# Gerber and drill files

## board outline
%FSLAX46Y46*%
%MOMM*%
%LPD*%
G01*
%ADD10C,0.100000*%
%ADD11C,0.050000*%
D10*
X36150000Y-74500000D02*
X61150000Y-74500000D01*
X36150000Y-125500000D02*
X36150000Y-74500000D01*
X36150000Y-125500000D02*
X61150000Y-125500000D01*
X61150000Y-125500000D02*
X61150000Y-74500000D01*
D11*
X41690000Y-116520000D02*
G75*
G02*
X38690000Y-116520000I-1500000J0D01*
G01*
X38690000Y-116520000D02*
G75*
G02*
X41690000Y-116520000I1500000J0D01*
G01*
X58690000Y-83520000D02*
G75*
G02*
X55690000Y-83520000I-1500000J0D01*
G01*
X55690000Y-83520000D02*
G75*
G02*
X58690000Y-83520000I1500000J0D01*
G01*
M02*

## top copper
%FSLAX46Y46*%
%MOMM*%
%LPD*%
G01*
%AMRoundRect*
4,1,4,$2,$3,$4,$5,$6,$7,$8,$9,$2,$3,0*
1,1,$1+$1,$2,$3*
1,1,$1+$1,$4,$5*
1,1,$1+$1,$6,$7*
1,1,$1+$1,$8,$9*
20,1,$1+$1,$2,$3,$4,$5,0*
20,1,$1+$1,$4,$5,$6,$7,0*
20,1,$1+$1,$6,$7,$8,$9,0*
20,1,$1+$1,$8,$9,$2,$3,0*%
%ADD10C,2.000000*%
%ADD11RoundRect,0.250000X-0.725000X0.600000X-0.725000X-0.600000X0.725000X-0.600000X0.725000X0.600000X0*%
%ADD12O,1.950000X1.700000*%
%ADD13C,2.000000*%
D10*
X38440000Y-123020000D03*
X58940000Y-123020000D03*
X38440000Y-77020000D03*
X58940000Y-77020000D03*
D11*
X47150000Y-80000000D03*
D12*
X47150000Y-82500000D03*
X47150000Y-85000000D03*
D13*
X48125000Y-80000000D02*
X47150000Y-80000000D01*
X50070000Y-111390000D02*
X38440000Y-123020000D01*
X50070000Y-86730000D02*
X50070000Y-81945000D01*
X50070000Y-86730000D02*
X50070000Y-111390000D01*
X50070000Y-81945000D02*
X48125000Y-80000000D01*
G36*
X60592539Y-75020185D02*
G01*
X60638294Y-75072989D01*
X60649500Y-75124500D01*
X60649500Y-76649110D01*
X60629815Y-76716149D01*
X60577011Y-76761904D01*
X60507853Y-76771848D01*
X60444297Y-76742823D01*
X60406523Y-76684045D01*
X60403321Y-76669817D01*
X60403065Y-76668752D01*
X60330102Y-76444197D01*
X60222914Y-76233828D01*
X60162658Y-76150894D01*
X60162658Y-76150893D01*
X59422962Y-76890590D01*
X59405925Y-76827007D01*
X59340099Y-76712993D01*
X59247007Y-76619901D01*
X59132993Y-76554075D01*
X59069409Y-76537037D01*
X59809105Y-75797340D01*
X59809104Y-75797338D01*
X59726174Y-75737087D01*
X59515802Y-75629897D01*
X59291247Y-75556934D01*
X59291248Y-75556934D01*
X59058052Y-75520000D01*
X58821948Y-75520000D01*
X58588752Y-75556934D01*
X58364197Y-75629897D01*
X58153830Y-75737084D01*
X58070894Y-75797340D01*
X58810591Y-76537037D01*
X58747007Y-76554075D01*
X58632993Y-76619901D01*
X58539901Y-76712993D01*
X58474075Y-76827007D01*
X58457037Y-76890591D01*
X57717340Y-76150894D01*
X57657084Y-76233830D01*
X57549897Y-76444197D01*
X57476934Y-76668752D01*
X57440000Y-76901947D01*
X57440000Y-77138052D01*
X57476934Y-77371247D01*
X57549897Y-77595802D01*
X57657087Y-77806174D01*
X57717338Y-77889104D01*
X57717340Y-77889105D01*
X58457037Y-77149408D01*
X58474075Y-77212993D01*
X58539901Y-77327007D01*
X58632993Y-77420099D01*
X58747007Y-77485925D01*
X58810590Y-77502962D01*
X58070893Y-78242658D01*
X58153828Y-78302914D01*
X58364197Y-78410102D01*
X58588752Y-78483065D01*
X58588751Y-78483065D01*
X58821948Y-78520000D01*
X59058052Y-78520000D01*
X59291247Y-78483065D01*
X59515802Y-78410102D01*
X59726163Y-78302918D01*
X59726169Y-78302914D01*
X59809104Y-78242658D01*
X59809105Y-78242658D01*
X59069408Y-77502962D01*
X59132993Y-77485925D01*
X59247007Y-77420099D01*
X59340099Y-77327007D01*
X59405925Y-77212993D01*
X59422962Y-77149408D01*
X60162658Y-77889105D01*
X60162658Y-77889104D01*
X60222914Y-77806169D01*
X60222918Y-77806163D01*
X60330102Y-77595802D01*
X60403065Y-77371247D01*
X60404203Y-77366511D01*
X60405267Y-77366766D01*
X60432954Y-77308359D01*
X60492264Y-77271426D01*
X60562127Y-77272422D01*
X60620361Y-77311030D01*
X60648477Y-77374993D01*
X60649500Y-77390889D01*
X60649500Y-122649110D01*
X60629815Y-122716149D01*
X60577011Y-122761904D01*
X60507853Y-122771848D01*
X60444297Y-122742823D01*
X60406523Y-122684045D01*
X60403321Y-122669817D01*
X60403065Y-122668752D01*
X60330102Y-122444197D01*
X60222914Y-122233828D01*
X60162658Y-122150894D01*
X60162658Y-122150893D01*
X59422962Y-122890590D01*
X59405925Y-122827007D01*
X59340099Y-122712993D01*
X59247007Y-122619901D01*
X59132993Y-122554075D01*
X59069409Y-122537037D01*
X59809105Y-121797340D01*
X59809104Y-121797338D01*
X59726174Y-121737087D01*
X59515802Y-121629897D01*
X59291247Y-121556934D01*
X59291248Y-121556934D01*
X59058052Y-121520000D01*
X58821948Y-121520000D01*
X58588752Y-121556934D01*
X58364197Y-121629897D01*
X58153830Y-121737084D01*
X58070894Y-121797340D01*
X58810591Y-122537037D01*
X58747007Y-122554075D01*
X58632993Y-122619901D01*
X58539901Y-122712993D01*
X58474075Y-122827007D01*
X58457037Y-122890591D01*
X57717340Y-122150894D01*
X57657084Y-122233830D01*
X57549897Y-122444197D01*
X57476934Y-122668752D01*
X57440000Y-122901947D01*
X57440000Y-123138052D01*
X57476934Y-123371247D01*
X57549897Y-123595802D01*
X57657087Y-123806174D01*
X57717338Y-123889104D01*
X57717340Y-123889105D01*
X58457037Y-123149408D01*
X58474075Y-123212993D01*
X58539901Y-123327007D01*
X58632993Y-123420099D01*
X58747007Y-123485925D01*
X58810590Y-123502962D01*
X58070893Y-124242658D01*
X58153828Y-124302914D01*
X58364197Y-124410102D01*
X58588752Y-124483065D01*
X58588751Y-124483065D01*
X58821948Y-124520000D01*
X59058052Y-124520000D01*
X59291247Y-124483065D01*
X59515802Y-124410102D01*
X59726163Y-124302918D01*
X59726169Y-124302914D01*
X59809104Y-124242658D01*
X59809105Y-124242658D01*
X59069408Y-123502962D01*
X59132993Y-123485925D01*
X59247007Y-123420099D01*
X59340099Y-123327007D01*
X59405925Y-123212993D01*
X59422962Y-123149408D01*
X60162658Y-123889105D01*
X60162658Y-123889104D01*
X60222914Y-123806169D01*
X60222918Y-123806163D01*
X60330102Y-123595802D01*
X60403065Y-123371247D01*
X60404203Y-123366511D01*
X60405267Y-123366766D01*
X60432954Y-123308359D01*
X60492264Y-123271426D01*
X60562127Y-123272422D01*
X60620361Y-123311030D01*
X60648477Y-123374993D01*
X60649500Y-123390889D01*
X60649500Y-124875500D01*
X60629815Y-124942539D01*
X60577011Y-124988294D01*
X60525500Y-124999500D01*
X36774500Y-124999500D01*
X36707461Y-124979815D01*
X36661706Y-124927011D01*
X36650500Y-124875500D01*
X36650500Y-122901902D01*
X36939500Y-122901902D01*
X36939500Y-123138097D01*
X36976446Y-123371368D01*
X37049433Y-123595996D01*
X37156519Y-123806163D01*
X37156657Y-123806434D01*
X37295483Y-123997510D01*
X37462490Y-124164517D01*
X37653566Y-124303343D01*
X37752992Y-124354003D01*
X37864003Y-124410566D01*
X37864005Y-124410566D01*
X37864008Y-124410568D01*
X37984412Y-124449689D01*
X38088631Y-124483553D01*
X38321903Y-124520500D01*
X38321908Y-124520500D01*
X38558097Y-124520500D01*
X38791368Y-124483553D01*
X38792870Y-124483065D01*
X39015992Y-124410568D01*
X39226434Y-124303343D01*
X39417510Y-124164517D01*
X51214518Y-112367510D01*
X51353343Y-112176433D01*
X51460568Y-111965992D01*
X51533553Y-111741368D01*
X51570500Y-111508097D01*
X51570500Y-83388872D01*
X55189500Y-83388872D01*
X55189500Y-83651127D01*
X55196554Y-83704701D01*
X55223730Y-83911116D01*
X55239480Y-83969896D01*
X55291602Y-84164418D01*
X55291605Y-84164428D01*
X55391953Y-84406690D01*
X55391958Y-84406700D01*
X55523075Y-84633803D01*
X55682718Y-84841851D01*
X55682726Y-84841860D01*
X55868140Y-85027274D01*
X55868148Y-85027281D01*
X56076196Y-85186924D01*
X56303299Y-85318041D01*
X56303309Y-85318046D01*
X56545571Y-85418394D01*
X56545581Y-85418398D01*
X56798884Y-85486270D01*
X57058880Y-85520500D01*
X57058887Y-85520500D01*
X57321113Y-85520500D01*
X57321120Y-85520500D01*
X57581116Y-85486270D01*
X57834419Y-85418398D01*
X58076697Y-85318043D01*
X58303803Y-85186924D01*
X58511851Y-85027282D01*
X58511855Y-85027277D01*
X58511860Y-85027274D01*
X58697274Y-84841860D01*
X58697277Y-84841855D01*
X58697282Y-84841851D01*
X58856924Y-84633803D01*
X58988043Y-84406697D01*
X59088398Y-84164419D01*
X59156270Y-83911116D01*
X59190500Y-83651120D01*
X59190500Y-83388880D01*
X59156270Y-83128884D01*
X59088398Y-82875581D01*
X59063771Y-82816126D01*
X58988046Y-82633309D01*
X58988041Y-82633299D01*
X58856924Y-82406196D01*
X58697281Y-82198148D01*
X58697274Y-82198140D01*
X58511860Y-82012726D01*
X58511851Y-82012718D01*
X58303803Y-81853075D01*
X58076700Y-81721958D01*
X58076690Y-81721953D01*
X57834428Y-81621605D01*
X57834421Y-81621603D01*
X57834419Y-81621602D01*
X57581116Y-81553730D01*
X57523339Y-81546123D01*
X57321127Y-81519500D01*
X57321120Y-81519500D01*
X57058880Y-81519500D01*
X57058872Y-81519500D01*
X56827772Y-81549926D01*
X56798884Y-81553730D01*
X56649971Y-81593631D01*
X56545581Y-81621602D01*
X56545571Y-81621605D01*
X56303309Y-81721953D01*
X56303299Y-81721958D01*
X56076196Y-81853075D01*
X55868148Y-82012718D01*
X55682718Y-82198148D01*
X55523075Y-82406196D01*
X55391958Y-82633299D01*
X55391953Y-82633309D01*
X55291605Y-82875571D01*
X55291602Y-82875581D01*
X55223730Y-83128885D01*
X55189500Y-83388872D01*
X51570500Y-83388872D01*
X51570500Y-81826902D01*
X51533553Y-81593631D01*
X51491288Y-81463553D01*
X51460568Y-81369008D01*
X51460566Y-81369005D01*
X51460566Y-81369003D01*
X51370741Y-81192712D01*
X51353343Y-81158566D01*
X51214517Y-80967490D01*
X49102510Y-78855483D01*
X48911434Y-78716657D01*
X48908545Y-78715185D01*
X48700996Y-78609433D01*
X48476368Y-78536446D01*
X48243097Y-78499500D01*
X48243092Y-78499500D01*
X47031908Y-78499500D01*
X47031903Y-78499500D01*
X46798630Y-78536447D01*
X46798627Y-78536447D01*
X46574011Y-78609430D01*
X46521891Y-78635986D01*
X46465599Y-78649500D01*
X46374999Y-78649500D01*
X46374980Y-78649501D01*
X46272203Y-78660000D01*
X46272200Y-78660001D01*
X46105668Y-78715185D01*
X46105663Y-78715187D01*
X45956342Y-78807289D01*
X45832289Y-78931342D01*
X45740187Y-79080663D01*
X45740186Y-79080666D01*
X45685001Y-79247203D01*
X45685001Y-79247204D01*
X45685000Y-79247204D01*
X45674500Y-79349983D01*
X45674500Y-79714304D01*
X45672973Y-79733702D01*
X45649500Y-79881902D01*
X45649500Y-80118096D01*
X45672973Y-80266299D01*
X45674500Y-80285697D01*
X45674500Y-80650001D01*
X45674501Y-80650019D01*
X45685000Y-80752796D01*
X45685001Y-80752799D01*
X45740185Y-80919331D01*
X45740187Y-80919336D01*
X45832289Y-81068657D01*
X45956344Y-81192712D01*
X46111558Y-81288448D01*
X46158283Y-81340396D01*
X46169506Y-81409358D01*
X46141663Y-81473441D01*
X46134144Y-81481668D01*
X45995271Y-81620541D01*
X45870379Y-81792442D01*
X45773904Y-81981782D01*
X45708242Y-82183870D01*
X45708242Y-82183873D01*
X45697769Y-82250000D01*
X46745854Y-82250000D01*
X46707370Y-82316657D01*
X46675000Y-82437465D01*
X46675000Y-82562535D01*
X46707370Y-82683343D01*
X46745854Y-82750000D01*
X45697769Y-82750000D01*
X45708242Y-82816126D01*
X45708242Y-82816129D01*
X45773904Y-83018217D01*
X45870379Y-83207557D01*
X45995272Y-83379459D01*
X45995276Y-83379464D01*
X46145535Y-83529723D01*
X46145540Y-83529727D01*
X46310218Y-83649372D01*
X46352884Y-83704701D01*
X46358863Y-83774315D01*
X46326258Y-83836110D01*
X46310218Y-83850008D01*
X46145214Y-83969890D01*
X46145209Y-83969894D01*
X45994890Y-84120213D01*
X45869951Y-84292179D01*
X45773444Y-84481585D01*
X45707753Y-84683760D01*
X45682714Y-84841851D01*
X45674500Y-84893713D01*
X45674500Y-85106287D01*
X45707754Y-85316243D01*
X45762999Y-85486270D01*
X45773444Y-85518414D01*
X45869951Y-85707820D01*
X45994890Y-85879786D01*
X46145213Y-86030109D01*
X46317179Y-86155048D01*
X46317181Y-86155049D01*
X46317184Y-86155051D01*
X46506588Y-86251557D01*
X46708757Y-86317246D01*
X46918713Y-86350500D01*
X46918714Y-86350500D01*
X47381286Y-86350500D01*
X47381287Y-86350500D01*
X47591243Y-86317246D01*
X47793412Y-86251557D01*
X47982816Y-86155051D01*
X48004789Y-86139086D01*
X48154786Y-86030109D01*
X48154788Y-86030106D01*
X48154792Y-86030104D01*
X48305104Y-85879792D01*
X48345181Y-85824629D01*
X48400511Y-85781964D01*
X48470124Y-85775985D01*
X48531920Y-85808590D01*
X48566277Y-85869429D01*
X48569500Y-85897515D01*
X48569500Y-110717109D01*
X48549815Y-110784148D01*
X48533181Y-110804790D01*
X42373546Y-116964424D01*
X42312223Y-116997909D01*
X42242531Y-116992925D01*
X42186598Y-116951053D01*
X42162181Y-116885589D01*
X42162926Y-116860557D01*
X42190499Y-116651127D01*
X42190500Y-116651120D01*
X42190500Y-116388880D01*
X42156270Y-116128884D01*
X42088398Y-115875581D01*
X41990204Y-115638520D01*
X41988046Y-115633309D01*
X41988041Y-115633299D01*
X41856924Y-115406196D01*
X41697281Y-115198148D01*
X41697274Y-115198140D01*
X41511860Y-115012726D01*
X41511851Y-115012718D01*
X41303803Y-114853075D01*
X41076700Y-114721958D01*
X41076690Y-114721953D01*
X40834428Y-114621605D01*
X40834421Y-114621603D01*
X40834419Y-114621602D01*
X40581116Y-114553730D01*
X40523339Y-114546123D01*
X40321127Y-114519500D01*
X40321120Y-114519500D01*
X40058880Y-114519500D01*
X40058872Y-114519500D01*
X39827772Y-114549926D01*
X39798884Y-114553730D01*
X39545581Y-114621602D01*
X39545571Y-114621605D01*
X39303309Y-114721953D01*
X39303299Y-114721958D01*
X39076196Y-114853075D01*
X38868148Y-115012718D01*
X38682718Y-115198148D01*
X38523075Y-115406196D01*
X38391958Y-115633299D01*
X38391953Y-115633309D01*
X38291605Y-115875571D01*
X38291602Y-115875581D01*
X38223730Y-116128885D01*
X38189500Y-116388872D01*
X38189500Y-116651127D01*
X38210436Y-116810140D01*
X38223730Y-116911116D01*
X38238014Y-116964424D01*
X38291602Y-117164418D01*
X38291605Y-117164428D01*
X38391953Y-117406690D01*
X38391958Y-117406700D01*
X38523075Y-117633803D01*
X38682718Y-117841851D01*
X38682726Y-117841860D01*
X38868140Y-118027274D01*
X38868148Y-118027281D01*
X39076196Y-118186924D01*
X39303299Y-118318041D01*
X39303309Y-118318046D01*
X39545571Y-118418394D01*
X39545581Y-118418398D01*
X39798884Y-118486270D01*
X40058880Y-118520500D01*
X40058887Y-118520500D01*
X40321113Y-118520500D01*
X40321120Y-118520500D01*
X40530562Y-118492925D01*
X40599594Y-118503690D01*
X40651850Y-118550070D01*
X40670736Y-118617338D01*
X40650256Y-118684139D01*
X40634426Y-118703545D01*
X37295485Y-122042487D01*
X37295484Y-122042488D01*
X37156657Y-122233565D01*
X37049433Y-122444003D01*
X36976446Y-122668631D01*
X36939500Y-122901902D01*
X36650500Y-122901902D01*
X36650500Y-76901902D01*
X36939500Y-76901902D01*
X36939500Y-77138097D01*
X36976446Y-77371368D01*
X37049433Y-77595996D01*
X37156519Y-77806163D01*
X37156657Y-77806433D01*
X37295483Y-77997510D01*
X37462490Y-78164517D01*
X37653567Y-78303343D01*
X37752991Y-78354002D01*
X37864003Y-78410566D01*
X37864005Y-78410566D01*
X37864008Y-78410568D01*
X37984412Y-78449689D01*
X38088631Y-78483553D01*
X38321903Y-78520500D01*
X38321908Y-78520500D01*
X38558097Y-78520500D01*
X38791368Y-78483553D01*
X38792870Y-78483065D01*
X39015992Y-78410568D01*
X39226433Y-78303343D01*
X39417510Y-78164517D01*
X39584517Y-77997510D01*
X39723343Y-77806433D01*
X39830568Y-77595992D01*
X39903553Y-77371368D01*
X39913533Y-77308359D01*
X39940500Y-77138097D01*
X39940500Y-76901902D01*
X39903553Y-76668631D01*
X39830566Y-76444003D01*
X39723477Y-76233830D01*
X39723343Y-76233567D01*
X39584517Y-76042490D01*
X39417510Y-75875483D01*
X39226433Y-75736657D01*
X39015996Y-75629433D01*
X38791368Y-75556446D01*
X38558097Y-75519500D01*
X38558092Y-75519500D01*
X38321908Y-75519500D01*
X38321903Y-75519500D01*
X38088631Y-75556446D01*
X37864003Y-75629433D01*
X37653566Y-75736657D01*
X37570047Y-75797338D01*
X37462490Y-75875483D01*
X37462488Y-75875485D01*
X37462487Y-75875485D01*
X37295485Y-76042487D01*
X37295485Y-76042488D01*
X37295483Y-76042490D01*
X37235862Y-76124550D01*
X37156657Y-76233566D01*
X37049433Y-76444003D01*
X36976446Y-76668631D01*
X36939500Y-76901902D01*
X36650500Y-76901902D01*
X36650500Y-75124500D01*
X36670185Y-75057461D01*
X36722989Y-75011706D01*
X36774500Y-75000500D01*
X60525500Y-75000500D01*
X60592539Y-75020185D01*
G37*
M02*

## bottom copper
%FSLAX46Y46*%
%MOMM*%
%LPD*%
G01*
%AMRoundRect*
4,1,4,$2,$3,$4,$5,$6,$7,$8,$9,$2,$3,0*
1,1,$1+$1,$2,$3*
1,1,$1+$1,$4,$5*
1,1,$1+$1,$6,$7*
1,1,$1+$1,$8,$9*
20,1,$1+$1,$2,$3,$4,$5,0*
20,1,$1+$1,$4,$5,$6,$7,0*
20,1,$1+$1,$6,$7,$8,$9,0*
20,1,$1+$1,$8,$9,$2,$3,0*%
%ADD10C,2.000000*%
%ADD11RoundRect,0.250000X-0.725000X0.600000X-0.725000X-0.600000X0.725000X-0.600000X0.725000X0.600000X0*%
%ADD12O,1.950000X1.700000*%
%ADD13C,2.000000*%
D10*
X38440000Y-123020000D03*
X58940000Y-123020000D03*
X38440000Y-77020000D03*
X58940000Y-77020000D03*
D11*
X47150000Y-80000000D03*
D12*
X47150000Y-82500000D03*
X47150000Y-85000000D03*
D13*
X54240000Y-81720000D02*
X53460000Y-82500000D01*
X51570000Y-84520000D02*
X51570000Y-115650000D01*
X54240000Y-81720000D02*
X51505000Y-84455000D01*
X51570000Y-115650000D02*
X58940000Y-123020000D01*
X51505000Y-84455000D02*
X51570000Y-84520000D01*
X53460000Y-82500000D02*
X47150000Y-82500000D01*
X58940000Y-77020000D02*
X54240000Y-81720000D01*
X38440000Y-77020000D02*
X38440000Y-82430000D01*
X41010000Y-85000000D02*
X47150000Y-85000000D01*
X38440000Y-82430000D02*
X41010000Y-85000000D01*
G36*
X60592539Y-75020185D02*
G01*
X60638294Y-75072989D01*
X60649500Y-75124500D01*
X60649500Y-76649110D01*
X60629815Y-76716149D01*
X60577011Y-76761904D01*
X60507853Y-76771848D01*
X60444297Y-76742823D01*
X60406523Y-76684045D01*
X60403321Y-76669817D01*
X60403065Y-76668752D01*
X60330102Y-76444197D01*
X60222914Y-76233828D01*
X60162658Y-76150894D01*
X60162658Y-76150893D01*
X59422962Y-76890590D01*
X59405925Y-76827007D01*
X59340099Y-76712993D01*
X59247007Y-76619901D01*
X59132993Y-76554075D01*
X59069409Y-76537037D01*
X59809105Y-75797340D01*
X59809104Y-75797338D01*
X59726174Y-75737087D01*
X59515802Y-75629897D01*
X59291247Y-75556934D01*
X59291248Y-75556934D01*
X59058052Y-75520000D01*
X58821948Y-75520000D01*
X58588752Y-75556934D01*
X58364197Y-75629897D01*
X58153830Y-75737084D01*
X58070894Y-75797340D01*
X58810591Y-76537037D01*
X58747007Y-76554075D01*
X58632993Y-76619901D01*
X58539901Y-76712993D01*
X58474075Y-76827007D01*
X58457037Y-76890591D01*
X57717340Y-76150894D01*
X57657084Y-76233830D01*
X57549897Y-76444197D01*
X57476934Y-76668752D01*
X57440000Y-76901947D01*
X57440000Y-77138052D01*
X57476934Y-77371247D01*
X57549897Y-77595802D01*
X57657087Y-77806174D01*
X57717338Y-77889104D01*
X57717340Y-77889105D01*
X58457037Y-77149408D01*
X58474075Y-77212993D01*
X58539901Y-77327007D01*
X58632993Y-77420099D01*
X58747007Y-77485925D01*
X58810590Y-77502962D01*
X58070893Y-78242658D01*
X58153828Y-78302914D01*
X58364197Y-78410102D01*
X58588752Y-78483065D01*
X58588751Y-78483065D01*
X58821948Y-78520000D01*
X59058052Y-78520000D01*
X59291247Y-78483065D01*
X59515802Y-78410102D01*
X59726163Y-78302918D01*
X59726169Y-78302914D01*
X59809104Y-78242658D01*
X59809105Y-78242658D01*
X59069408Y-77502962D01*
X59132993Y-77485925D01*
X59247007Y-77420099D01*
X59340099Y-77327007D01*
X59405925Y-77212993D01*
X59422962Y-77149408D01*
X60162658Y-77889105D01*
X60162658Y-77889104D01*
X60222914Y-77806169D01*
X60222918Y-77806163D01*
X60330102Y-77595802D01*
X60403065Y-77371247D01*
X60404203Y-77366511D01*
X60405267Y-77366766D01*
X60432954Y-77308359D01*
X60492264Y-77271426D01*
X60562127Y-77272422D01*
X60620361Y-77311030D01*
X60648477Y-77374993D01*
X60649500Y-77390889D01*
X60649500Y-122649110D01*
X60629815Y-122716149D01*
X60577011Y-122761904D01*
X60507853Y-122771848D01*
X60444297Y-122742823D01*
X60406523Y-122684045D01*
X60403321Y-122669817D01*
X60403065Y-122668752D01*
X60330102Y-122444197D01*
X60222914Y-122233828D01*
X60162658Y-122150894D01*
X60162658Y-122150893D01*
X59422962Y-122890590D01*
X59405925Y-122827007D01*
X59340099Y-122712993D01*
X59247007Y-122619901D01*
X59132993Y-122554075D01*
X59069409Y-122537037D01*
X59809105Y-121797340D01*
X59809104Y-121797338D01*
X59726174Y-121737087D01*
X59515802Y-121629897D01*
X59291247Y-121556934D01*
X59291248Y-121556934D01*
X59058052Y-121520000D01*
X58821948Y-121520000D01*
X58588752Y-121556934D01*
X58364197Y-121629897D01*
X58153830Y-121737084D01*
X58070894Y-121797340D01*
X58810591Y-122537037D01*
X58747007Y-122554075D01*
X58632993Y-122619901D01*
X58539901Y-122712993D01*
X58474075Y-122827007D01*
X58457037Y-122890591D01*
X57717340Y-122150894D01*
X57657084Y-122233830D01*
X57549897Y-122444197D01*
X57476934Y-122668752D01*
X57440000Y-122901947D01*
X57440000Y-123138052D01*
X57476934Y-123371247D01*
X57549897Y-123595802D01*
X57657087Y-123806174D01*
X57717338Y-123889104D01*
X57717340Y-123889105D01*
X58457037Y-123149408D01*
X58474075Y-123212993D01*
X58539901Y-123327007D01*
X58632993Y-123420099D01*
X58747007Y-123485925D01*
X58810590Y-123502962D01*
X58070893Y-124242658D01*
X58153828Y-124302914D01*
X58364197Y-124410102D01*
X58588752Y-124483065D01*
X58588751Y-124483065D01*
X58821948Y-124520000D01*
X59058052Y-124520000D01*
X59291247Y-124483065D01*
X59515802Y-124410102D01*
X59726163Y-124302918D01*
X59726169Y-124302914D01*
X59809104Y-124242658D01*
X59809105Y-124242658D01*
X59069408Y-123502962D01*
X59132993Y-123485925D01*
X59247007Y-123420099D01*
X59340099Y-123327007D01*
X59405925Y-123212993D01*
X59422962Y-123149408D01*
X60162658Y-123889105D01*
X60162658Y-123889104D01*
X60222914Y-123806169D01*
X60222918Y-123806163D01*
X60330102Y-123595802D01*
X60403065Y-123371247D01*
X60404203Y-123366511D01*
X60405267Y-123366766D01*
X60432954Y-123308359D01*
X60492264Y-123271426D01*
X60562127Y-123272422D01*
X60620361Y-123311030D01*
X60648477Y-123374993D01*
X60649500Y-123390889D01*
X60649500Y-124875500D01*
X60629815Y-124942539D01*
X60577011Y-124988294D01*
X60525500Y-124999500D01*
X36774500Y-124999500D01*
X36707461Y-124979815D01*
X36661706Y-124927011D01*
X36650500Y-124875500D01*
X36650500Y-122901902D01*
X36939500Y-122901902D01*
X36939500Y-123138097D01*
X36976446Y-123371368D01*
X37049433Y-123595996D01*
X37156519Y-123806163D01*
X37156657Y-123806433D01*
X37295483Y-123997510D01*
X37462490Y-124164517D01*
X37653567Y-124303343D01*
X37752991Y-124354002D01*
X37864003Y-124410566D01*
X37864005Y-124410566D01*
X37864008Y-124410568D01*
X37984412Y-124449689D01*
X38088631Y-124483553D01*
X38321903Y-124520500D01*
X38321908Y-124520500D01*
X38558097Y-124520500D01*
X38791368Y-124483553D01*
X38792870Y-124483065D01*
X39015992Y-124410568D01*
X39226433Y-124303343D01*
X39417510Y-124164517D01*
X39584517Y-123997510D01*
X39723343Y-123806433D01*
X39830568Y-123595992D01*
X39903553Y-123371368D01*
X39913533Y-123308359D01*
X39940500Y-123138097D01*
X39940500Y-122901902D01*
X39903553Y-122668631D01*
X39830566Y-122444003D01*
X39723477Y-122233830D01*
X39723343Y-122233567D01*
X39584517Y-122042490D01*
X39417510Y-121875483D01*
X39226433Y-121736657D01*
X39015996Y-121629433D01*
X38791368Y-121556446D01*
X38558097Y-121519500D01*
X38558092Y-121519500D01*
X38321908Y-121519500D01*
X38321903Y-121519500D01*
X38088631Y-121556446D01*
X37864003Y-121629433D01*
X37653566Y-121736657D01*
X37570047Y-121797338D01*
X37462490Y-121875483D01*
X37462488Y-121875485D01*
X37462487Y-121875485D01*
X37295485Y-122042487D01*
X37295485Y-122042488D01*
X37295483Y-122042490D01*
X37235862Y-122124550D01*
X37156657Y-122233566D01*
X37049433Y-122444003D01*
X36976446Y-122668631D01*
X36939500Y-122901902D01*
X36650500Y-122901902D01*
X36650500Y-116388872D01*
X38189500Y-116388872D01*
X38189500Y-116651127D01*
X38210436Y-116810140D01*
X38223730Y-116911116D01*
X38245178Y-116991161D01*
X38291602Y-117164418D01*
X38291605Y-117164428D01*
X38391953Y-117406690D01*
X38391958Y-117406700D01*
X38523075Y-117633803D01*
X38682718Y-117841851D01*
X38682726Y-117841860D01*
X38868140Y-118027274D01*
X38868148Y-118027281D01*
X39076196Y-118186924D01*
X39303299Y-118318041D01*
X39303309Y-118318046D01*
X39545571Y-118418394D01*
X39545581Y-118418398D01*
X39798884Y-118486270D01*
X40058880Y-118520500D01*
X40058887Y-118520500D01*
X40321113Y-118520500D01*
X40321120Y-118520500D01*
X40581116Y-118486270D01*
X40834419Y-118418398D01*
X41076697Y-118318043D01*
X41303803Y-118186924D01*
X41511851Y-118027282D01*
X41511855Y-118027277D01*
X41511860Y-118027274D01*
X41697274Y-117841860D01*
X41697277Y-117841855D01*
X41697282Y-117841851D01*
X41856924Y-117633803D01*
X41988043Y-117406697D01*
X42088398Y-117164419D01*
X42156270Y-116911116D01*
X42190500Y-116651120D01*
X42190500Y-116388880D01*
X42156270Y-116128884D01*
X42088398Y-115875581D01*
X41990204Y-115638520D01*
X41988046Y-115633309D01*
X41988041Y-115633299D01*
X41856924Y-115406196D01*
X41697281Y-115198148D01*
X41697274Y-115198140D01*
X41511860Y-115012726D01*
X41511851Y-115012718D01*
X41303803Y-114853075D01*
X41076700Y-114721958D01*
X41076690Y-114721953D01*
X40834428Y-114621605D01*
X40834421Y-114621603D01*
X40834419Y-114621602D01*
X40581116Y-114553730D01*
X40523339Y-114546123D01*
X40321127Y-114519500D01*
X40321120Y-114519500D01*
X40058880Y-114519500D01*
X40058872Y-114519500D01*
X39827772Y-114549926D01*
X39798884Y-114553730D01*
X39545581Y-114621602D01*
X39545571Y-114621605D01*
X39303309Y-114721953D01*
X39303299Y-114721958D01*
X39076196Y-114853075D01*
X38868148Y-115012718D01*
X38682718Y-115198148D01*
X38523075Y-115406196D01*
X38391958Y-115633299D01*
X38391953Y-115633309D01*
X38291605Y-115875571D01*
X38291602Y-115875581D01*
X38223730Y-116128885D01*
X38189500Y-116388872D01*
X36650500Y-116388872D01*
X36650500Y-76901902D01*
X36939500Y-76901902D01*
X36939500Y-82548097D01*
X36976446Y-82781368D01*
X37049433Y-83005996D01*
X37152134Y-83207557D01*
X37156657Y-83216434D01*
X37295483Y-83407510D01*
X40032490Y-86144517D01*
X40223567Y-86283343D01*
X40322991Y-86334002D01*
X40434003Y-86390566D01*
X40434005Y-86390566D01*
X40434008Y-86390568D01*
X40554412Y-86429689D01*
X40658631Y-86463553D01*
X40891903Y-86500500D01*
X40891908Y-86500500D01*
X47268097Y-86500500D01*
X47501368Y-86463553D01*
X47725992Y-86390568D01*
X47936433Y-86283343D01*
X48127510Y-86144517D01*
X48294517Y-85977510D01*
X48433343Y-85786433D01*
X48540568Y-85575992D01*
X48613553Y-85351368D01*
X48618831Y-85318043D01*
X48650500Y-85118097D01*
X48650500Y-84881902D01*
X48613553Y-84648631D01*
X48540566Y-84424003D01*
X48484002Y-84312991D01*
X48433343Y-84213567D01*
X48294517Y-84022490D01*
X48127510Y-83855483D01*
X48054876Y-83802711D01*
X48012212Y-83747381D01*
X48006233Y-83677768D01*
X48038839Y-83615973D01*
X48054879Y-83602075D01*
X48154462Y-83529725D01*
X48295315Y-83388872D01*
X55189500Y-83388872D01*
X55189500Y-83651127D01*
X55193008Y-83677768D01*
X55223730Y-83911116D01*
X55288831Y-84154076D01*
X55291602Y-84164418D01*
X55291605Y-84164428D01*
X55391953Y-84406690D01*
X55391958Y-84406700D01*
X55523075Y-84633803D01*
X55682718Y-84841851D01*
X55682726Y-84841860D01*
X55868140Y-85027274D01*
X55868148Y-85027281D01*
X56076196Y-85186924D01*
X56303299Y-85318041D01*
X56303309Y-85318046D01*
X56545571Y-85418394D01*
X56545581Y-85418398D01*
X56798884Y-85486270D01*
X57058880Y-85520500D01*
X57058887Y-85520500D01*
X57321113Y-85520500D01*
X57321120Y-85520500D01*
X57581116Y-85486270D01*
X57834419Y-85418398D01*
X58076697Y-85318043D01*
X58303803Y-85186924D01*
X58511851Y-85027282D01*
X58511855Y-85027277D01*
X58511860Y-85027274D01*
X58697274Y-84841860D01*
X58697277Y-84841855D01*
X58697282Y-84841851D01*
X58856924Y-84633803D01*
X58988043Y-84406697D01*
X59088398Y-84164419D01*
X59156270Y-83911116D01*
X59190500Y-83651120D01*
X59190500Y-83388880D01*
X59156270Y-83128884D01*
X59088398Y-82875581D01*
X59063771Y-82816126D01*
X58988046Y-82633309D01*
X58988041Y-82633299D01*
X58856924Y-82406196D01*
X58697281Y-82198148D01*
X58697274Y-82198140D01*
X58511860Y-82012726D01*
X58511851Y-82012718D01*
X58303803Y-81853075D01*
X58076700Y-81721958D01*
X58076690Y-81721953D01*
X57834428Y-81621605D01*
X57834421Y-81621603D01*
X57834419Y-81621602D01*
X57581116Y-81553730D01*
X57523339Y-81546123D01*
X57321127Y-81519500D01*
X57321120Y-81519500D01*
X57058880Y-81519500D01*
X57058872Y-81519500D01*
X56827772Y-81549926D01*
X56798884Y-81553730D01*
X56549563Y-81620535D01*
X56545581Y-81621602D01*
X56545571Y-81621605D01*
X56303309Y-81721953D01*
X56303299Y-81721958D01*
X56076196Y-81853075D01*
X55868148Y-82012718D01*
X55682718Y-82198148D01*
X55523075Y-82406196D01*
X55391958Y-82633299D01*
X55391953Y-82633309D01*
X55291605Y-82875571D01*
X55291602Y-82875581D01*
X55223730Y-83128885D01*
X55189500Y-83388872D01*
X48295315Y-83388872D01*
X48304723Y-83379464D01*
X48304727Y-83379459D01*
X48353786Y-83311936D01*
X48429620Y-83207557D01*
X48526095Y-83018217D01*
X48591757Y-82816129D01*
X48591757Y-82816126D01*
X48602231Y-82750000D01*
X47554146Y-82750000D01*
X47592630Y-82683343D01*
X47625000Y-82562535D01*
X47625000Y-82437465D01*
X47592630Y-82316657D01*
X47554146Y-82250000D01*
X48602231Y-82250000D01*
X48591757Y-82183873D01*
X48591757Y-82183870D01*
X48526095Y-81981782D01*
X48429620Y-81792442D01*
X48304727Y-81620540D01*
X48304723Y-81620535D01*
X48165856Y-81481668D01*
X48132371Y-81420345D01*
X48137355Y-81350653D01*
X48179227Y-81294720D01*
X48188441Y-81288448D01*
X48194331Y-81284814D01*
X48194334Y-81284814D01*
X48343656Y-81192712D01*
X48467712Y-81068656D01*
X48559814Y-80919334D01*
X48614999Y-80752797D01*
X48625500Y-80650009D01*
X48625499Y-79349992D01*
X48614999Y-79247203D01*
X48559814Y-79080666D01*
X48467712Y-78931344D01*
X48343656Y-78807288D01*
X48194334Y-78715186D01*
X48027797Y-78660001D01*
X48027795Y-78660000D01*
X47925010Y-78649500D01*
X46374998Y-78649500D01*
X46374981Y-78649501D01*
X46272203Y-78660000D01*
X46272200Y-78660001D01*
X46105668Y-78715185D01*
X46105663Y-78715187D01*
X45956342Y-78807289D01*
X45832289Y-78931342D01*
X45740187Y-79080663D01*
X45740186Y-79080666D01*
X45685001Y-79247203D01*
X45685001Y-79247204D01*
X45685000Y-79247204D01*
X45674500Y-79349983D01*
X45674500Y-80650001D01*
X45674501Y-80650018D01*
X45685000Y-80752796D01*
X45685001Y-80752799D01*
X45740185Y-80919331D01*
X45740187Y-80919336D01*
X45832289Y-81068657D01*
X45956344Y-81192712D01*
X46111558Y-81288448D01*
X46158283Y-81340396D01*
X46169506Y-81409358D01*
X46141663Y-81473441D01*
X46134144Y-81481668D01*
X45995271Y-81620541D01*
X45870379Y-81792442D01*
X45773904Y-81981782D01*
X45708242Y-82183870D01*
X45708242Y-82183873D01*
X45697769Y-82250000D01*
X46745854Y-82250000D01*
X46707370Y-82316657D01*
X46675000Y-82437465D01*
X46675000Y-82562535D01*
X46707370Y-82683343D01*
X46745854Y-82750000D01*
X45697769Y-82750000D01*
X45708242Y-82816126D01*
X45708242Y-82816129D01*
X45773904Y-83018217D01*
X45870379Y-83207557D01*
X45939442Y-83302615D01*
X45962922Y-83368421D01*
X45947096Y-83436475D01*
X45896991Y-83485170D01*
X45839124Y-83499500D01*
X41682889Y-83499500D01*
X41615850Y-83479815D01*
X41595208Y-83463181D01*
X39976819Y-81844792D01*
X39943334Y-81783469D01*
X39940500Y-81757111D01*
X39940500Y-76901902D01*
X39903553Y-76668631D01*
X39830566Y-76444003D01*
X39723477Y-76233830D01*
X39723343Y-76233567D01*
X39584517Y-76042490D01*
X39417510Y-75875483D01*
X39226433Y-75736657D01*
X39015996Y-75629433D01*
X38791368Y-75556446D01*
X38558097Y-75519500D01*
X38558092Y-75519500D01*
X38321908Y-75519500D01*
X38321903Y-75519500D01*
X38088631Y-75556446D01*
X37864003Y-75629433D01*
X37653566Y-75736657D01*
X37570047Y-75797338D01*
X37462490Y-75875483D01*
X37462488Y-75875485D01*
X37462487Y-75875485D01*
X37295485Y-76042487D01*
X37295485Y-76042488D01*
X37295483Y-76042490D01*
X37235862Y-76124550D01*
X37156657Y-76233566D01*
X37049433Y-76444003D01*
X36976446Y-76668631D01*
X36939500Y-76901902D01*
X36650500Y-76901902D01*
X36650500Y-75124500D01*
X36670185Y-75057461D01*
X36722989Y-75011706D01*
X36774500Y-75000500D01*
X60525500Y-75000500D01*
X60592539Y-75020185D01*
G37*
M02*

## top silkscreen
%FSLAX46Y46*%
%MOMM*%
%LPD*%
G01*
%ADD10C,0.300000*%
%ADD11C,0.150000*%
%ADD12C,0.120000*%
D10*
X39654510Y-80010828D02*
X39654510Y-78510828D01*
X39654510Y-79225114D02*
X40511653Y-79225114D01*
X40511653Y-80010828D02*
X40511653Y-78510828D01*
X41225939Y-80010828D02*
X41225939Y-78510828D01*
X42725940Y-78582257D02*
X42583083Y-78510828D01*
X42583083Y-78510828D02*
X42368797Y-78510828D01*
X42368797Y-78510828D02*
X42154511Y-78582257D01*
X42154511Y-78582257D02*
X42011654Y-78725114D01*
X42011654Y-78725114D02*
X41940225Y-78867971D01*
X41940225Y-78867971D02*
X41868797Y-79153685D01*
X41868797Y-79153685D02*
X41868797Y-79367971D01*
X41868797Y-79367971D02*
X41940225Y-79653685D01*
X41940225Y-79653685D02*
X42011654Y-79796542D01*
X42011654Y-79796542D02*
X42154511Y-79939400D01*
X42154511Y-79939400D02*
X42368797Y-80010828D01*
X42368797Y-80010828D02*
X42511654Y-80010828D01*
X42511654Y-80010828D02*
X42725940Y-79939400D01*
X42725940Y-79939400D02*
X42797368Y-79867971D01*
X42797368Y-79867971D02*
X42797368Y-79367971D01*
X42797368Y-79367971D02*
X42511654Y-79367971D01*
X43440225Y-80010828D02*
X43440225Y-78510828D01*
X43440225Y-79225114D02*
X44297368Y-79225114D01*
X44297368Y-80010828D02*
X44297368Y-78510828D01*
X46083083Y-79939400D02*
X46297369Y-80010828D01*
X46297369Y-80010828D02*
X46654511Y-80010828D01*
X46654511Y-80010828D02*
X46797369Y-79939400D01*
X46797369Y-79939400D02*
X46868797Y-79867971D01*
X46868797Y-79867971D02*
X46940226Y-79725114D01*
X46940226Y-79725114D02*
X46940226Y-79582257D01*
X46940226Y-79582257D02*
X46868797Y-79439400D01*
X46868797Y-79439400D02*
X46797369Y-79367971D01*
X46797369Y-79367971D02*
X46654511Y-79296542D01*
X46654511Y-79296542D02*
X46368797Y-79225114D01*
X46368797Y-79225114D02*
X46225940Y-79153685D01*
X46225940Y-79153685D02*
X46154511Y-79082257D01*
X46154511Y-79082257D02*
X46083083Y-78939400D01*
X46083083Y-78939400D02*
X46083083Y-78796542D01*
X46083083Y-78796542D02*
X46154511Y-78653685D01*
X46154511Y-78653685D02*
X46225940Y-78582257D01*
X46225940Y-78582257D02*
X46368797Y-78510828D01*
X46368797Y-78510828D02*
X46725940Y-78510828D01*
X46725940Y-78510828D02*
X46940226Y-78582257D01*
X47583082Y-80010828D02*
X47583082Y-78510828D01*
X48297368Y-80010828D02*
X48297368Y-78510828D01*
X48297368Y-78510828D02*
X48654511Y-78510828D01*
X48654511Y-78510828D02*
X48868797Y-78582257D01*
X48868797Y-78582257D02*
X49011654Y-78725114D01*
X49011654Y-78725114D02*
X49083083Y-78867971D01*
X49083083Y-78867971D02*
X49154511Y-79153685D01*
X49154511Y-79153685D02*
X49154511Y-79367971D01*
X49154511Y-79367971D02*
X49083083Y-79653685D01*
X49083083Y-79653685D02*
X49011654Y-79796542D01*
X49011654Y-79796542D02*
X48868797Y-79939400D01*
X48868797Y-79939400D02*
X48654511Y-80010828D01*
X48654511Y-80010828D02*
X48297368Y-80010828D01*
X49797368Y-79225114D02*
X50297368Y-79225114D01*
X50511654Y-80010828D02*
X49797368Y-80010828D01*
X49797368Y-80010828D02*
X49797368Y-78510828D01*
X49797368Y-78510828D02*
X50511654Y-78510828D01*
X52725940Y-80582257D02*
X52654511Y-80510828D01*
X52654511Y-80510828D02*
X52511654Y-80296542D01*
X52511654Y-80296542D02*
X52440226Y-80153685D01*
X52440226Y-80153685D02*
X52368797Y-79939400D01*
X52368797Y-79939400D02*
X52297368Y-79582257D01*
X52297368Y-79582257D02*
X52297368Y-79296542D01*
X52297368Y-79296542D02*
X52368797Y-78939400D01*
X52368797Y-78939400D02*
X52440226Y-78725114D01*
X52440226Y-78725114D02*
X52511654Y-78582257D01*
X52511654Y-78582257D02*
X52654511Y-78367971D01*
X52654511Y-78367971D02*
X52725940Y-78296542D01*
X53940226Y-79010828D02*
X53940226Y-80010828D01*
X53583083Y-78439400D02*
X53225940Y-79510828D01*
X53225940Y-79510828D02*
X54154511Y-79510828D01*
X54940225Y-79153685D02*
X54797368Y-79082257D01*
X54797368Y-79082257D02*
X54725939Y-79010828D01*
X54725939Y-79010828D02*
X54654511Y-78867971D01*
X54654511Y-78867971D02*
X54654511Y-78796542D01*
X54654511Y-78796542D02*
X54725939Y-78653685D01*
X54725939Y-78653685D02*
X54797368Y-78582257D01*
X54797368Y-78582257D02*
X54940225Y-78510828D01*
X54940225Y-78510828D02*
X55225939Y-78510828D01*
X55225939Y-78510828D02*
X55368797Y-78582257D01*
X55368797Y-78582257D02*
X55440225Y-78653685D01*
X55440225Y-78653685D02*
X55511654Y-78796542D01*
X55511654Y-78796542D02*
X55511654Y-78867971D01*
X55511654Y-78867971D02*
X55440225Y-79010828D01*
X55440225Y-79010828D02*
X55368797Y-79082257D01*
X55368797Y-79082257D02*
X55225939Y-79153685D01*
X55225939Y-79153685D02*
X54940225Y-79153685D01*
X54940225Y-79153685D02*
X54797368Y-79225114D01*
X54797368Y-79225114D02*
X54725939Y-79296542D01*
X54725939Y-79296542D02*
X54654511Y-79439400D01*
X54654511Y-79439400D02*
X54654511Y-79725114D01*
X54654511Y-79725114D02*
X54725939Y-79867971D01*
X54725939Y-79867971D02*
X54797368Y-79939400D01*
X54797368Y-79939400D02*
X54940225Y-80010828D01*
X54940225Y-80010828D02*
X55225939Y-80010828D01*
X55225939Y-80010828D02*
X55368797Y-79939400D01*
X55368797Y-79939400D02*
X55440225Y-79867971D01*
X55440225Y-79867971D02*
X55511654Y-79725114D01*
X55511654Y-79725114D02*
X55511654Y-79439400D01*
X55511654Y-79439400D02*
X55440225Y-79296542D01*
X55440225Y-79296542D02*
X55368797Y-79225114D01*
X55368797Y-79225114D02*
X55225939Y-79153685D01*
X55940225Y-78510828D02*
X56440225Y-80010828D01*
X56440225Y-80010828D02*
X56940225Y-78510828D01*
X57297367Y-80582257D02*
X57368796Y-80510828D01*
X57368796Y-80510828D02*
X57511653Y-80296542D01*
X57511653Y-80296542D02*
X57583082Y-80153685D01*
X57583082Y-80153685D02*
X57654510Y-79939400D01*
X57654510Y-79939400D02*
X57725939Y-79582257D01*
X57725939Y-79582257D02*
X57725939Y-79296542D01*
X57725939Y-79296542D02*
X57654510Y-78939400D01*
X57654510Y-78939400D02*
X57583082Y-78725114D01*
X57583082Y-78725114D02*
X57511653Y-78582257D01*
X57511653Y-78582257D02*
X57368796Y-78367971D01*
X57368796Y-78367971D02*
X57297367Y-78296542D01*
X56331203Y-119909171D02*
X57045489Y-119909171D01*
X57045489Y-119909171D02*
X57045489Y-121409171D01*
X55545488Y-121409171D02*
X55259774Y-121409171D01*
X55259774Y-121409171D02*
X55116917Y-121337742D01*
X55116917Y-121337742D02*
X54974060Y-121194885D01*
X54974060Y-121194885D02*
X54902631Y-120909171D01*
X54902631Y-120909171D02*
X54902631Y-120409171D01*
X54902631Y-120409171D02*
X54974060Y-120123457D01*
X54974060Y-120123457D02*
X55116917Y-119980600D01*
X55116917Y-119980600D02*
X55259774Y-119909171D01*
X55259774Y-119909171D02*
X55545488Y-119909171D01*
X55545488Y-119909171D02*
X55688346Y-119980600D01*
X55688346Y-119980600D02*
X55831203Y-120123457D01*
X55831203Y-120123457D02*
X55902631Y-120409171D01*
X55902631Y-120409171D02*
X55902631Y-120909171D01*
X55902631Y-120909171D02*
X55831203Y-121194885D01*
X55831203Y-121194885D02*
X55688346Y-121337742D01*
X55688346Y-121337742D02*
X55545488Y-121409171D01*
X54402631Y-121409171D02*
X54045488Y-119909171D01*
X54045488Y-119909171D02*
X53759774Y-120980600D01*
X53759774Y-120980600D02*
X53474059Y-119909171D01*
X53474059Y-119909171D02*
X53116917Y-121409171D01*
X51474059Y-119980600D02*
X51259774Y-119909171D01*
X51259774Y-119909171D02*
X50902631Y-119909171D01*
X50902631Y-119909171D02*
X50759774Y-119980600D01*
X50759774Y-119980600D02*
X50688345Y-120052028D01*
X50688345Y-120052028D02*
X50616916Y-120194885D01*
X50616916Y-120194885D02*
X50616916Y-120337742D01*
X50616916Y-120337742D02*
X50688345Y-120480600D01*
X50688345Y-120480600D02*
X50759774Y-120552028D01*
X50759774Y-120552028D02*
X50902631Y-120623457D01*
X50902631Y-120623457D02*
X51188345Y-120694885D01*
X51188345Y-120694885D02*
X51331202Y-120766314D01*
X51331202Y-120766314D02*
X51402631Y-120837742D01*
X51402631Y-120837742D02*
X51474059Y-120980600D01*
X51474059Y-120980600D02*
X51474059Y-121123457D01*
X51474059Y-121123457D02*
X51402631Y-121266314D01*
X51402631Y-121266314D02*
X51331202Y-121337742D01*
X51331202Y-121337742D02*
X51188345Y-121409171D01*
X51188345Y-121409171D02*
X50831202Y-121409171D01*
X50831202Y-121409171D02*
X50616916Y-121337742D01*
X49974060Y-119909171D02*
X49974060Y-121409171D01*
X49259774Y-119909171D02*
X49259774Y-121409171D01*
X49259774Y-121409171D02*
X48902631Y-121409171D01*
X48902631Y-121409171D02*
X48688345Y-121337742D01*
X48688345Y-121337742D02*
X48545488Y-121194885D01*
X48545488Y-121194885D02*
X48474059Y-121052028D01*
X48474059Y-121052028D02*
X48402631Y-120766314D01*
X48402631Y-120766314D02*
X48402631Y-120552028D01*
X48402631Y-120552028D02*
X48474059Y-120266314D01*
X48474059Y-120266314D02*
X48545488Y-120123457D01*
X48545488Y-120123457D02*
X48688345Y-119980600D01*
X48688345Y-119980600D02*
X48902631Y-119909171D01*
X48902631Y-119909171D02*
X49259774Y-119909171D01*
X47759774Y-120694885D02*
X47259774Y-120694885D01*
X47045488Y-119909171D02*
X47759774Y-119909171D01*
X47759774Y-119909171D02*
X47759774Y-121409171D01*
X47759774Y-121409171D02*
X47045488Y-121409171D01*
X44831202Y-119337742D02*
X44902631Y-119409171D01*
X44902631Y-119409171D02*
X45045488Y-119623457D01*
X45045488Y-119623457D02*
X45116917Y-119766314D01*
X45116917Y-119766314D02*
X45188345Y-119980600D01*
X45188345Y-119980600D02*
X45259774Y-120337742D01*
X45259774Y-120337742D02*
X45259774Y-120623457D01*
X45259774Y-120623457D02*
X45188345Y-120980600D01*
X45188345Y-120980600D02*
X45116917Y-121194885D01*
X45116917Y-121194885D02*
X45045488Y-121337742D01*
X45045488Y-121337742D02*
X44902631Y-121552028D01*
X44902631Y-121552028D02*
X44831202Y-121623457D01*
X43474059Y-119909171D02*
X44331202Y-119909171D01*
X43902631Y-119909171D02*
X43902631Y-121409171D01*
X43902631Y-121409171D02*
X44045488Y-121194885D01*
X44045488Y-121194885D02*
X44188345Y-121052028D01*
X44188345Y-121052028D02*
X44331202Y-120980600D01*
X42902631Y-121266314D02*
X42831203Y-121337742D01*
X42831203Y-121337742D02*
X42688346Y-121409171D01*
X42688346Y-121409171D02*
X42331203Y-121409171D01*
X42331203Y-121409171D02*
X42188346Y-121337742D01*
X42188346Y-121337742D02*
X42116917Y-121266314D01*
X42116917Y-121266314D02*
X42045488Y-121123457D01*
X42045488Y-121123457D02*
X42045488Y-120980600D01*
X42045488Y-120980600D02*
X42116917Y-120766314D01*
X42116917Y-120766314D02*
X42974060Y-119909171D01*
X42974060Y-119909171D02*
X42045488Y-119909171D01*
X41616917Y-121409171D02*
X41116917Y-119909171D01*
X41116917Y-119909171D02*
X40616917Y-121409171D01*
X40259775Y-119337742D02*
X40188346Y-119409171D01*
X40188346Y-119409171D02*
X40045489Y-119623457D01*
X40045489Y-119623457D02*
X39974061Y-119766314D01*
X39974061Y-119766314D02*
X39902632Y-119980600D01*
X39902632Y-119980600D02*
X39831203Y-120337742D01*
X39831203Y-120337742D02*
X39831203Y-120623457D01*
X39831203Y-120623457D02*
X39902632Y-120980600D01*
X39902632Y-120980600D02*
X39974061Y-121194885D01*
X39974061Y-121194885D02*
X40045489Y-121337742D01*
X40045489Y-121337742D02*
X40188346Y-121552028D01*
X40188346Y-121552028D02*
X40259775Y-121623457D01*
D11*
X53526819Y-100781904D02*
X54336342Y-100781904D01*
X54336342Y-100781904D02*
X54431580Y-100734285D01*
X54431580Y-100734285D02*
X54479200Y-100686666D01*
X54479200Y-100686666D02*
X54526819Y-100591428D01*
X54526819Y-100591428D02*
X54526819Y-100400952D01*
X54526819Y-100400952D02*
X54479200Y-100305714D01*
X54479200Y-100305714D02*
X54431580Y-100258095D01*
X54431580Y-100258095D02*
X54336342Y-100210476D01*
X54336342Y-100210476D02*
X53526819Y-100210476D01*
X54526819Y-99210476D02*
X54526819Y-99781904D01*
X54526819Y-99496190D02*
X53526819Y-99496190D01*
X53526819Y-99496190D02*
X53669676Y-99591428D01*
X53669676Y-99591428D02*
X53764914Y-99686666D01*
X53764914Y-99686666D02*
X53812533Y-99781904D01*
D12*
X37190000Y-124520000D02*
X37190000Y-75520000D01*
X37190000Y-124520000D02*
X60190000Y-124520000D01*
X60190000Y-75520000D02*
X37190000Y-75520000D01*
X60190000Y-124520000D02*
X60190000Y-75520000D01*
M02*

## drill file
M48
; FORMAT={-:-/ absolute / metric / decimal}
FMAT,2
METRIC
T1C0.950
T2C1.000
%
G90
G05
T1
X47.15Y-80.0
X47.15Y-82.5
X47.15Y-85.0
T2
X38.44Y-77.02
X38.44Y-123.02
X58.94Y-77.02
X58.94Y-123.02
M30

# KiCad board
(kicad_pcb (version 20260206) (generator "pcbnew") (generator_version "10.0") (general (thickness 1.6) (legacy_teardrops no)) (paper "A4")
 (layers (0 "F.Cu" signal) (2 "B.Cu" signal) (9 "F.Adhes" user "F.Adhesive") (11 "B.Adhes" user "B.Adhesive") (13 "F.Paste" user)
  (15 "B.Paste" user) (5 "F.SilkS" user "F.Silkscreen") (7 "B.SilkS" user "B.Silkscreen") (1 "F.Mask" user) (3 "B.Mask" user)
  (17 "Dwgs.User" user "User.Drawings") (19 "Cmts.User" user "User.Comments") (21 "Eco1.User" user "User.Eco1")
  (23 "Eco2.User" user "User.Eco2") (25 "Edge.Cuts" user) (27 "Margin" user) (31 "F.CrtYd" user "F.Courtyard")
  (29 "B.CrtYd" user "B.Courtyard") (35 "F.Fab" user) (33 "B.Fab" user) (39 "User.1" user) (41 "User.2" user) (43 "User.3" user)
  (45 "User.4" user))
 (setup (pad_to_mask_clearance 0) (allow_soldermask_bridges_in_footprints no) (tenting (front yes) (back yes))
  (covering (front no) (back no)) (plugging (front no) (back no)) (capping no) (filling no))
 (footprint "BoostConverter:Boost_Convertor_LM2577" (layer "F.Cu") (at 48.69 100.02 90)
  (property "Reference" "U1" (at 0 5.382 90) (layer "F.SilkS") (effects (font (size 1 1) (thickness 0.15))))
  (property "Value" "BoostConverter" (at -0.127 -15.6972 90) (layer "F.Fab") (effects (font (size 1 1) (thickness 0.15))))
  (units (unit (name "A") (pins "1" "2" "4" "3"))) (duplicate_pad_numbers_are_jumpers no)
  (fp_line (start -24.5 -11.5) (end 24.5 -11.5) (stroke (width 0.12) (type solid)) (layer "F.SilkS"))
  (fp_line (start -24.5 -11.5) (end -24.5 11.5) (stroke (width 0.12) (type solid)) (layer "F.SilkS"))
  (fp_line (start 24.5 11.5) (end 24.5 -11.5) (stroke (width 0.12) (type solid)) (layer "F.SilkS"))
  (fp_line (start -24.5 11.5) (end 24.5 11.5) (stroke (width 0.12) (type solid)) (layer "F.SilkS"))
  (fp_circle (center -16.5 -8.5) (end -15 -8.5) (stroke (width 0.05) (type default)) (fill no) (layer "Edge.Cuts"))
  (fp_circle (center 16.5 8.5) (end 18 8.5) (stroke (width 0.05) (type default)) (fill no) (layer "Edge.Cuts"))
  (pad "1" thru_hole circle (at -23 -10.25 90) (size 2 2) (drill 1) (layers "*.Cu" "*.Mask") (remove_unused_layers no) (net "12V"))
  (pad "2" thru_hole circle (at -23 10.25 90) (size 2 2) (drill 1) (layers "*.Cu" "*.Mask") (remove_unused_layers no) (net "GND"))
  (pad "3" thru_hole circle (at 23 -10.25 90) (size 2 2) (drill 1) (layers "*.Cu" "*.Mask") (remove_unused_layers no) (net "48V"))
  (pad "4" thru_hole circle (at 23 10.25 90) (size 2 2) (drill 1) (layers "*.Cu" "*.Mask") (remove_unused_layers no) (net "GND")))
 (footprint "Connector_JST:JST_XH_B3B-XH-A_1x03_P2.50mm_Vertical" (layer "B.Cu") (at 47.15 80 -90)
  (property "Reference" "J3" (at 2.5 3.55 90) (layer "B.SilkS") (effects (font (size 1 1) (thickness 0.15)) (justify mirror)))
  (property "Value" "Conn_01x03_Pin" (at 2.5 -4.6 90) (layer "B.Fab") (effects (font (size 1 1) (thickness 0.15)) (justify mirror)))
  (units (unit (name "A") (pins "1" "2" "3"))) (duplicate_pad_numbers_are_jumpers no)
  (pad "1" thru_hole roundrect (at 0 0 270) (size 1.7 1.95) (drill 0.95) (layers "*.Cu" "*.Mask") (remove_unused_layers no)
   (roundrect_rratio 0.147059) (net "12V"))
  (pad "2" thru_hole oval (at 2.5 0 270) (size 1.7 1.95) (drill 0.95) (layers "*.Cu" "*.Mask") (remove_unused_layers no) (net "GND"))
  (pad "3" thru_hole oval (at 5 0 270) (size 1.7 1.95) (drill 0.95) (layers "*.Cu" "*.Mask") (remove_unused_layers no) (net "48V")))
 (gr_line (start 36.15 74.5) (end 61.15 74.5) (stroke (width 0.1) (type default)) (layer "Edge.Cuts"))
 (gr_line (start 36.15 125.5) (end 36.15 74.5) (stroke (width 0.1) (type default)) (layer "Edge.Cuts"))
 (gr_line (start 36.15 125.5) (end 61.15 125.5) (stroke (width 0.1) (type default)) (layer "Edge.Cuts"))
 (gr_line (start 61.15 125.5) (end 61.15 74.5) (stroke (width 0.1) (type default)) (layer "Edge.Cuts"))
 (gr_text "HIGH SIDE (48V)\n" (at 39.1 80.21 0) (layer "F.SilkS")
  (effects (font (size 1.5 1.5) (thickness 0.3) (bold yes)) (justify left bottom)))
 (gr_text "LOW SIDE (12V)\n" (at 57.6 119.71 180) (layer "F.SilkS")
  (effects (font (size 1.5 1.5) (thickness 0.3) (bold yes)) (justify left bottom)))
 (segment (start 48.125 80) (end 47.15 80) (width 2) (layer "F.Cu") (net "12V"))
 (segment (start 50.07 111.39) (end 38.44 123.02) (width 2) (layer "F.Cu") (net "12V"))
 (segment (start 50.07 86.73) (end 50.07 81.945) (width 2) (layer "F.Cu") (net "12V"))
 (segment (start 50.07 86.73) (end 50.07 111.39) (width 2) (layer "F.Cu") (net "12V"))
 (segment (start 50.07 81.945) (end 48.125 80) (width 2) (layer "F.Cu") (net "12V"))
 (segment (start 54.24 81.72) (end 53.46 82.5) (width 2) (layer "B.Cu") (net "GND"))
 (segment (start 51.57 84.52) (end 51.57 115.65) (width 2) (layer "B.Cu") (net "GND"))
 (segment (start 54.24 81.72) (end 51.505 84.455) (width 2) (layer "B.Cu") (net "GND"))
 (segment (start 51.57 115.65) (end 58.94 123.02) (width 2) (layer "B.Cu") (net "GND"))
 (segment (start 51.505 84.455) (end 51.57 84.52) (width 2) (layer "B.Cu") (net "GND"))
 (segment (start 53.46 82.5) (end 47.15 82.5) (width 2) (layer "B.Cu") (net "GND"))
 (segment (start 58.94 77.02) (end 54.24 81.72) (width 2) (layer "B.Cu") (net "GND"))
 (segment (start 38.44 77.02) (end 38.44 82.43) (width 2) (layer "B.Cu") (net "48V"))
 (segment (start 41.01 85) (end 47.15 85) (width 2) (layer "B.Cu") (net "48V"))
 (segment (start 38.44 82.43) (end 41.01 85) (width 2) (layer "B.Cu") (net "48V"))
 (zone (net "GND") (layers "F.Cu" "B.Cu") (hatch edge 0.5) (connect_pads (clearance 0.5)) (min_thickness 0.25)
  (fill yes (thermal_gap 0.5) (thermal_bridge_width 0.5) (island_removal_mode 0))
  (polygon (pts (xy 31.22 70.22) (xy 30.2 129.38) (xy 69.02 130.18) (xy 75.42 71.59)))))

